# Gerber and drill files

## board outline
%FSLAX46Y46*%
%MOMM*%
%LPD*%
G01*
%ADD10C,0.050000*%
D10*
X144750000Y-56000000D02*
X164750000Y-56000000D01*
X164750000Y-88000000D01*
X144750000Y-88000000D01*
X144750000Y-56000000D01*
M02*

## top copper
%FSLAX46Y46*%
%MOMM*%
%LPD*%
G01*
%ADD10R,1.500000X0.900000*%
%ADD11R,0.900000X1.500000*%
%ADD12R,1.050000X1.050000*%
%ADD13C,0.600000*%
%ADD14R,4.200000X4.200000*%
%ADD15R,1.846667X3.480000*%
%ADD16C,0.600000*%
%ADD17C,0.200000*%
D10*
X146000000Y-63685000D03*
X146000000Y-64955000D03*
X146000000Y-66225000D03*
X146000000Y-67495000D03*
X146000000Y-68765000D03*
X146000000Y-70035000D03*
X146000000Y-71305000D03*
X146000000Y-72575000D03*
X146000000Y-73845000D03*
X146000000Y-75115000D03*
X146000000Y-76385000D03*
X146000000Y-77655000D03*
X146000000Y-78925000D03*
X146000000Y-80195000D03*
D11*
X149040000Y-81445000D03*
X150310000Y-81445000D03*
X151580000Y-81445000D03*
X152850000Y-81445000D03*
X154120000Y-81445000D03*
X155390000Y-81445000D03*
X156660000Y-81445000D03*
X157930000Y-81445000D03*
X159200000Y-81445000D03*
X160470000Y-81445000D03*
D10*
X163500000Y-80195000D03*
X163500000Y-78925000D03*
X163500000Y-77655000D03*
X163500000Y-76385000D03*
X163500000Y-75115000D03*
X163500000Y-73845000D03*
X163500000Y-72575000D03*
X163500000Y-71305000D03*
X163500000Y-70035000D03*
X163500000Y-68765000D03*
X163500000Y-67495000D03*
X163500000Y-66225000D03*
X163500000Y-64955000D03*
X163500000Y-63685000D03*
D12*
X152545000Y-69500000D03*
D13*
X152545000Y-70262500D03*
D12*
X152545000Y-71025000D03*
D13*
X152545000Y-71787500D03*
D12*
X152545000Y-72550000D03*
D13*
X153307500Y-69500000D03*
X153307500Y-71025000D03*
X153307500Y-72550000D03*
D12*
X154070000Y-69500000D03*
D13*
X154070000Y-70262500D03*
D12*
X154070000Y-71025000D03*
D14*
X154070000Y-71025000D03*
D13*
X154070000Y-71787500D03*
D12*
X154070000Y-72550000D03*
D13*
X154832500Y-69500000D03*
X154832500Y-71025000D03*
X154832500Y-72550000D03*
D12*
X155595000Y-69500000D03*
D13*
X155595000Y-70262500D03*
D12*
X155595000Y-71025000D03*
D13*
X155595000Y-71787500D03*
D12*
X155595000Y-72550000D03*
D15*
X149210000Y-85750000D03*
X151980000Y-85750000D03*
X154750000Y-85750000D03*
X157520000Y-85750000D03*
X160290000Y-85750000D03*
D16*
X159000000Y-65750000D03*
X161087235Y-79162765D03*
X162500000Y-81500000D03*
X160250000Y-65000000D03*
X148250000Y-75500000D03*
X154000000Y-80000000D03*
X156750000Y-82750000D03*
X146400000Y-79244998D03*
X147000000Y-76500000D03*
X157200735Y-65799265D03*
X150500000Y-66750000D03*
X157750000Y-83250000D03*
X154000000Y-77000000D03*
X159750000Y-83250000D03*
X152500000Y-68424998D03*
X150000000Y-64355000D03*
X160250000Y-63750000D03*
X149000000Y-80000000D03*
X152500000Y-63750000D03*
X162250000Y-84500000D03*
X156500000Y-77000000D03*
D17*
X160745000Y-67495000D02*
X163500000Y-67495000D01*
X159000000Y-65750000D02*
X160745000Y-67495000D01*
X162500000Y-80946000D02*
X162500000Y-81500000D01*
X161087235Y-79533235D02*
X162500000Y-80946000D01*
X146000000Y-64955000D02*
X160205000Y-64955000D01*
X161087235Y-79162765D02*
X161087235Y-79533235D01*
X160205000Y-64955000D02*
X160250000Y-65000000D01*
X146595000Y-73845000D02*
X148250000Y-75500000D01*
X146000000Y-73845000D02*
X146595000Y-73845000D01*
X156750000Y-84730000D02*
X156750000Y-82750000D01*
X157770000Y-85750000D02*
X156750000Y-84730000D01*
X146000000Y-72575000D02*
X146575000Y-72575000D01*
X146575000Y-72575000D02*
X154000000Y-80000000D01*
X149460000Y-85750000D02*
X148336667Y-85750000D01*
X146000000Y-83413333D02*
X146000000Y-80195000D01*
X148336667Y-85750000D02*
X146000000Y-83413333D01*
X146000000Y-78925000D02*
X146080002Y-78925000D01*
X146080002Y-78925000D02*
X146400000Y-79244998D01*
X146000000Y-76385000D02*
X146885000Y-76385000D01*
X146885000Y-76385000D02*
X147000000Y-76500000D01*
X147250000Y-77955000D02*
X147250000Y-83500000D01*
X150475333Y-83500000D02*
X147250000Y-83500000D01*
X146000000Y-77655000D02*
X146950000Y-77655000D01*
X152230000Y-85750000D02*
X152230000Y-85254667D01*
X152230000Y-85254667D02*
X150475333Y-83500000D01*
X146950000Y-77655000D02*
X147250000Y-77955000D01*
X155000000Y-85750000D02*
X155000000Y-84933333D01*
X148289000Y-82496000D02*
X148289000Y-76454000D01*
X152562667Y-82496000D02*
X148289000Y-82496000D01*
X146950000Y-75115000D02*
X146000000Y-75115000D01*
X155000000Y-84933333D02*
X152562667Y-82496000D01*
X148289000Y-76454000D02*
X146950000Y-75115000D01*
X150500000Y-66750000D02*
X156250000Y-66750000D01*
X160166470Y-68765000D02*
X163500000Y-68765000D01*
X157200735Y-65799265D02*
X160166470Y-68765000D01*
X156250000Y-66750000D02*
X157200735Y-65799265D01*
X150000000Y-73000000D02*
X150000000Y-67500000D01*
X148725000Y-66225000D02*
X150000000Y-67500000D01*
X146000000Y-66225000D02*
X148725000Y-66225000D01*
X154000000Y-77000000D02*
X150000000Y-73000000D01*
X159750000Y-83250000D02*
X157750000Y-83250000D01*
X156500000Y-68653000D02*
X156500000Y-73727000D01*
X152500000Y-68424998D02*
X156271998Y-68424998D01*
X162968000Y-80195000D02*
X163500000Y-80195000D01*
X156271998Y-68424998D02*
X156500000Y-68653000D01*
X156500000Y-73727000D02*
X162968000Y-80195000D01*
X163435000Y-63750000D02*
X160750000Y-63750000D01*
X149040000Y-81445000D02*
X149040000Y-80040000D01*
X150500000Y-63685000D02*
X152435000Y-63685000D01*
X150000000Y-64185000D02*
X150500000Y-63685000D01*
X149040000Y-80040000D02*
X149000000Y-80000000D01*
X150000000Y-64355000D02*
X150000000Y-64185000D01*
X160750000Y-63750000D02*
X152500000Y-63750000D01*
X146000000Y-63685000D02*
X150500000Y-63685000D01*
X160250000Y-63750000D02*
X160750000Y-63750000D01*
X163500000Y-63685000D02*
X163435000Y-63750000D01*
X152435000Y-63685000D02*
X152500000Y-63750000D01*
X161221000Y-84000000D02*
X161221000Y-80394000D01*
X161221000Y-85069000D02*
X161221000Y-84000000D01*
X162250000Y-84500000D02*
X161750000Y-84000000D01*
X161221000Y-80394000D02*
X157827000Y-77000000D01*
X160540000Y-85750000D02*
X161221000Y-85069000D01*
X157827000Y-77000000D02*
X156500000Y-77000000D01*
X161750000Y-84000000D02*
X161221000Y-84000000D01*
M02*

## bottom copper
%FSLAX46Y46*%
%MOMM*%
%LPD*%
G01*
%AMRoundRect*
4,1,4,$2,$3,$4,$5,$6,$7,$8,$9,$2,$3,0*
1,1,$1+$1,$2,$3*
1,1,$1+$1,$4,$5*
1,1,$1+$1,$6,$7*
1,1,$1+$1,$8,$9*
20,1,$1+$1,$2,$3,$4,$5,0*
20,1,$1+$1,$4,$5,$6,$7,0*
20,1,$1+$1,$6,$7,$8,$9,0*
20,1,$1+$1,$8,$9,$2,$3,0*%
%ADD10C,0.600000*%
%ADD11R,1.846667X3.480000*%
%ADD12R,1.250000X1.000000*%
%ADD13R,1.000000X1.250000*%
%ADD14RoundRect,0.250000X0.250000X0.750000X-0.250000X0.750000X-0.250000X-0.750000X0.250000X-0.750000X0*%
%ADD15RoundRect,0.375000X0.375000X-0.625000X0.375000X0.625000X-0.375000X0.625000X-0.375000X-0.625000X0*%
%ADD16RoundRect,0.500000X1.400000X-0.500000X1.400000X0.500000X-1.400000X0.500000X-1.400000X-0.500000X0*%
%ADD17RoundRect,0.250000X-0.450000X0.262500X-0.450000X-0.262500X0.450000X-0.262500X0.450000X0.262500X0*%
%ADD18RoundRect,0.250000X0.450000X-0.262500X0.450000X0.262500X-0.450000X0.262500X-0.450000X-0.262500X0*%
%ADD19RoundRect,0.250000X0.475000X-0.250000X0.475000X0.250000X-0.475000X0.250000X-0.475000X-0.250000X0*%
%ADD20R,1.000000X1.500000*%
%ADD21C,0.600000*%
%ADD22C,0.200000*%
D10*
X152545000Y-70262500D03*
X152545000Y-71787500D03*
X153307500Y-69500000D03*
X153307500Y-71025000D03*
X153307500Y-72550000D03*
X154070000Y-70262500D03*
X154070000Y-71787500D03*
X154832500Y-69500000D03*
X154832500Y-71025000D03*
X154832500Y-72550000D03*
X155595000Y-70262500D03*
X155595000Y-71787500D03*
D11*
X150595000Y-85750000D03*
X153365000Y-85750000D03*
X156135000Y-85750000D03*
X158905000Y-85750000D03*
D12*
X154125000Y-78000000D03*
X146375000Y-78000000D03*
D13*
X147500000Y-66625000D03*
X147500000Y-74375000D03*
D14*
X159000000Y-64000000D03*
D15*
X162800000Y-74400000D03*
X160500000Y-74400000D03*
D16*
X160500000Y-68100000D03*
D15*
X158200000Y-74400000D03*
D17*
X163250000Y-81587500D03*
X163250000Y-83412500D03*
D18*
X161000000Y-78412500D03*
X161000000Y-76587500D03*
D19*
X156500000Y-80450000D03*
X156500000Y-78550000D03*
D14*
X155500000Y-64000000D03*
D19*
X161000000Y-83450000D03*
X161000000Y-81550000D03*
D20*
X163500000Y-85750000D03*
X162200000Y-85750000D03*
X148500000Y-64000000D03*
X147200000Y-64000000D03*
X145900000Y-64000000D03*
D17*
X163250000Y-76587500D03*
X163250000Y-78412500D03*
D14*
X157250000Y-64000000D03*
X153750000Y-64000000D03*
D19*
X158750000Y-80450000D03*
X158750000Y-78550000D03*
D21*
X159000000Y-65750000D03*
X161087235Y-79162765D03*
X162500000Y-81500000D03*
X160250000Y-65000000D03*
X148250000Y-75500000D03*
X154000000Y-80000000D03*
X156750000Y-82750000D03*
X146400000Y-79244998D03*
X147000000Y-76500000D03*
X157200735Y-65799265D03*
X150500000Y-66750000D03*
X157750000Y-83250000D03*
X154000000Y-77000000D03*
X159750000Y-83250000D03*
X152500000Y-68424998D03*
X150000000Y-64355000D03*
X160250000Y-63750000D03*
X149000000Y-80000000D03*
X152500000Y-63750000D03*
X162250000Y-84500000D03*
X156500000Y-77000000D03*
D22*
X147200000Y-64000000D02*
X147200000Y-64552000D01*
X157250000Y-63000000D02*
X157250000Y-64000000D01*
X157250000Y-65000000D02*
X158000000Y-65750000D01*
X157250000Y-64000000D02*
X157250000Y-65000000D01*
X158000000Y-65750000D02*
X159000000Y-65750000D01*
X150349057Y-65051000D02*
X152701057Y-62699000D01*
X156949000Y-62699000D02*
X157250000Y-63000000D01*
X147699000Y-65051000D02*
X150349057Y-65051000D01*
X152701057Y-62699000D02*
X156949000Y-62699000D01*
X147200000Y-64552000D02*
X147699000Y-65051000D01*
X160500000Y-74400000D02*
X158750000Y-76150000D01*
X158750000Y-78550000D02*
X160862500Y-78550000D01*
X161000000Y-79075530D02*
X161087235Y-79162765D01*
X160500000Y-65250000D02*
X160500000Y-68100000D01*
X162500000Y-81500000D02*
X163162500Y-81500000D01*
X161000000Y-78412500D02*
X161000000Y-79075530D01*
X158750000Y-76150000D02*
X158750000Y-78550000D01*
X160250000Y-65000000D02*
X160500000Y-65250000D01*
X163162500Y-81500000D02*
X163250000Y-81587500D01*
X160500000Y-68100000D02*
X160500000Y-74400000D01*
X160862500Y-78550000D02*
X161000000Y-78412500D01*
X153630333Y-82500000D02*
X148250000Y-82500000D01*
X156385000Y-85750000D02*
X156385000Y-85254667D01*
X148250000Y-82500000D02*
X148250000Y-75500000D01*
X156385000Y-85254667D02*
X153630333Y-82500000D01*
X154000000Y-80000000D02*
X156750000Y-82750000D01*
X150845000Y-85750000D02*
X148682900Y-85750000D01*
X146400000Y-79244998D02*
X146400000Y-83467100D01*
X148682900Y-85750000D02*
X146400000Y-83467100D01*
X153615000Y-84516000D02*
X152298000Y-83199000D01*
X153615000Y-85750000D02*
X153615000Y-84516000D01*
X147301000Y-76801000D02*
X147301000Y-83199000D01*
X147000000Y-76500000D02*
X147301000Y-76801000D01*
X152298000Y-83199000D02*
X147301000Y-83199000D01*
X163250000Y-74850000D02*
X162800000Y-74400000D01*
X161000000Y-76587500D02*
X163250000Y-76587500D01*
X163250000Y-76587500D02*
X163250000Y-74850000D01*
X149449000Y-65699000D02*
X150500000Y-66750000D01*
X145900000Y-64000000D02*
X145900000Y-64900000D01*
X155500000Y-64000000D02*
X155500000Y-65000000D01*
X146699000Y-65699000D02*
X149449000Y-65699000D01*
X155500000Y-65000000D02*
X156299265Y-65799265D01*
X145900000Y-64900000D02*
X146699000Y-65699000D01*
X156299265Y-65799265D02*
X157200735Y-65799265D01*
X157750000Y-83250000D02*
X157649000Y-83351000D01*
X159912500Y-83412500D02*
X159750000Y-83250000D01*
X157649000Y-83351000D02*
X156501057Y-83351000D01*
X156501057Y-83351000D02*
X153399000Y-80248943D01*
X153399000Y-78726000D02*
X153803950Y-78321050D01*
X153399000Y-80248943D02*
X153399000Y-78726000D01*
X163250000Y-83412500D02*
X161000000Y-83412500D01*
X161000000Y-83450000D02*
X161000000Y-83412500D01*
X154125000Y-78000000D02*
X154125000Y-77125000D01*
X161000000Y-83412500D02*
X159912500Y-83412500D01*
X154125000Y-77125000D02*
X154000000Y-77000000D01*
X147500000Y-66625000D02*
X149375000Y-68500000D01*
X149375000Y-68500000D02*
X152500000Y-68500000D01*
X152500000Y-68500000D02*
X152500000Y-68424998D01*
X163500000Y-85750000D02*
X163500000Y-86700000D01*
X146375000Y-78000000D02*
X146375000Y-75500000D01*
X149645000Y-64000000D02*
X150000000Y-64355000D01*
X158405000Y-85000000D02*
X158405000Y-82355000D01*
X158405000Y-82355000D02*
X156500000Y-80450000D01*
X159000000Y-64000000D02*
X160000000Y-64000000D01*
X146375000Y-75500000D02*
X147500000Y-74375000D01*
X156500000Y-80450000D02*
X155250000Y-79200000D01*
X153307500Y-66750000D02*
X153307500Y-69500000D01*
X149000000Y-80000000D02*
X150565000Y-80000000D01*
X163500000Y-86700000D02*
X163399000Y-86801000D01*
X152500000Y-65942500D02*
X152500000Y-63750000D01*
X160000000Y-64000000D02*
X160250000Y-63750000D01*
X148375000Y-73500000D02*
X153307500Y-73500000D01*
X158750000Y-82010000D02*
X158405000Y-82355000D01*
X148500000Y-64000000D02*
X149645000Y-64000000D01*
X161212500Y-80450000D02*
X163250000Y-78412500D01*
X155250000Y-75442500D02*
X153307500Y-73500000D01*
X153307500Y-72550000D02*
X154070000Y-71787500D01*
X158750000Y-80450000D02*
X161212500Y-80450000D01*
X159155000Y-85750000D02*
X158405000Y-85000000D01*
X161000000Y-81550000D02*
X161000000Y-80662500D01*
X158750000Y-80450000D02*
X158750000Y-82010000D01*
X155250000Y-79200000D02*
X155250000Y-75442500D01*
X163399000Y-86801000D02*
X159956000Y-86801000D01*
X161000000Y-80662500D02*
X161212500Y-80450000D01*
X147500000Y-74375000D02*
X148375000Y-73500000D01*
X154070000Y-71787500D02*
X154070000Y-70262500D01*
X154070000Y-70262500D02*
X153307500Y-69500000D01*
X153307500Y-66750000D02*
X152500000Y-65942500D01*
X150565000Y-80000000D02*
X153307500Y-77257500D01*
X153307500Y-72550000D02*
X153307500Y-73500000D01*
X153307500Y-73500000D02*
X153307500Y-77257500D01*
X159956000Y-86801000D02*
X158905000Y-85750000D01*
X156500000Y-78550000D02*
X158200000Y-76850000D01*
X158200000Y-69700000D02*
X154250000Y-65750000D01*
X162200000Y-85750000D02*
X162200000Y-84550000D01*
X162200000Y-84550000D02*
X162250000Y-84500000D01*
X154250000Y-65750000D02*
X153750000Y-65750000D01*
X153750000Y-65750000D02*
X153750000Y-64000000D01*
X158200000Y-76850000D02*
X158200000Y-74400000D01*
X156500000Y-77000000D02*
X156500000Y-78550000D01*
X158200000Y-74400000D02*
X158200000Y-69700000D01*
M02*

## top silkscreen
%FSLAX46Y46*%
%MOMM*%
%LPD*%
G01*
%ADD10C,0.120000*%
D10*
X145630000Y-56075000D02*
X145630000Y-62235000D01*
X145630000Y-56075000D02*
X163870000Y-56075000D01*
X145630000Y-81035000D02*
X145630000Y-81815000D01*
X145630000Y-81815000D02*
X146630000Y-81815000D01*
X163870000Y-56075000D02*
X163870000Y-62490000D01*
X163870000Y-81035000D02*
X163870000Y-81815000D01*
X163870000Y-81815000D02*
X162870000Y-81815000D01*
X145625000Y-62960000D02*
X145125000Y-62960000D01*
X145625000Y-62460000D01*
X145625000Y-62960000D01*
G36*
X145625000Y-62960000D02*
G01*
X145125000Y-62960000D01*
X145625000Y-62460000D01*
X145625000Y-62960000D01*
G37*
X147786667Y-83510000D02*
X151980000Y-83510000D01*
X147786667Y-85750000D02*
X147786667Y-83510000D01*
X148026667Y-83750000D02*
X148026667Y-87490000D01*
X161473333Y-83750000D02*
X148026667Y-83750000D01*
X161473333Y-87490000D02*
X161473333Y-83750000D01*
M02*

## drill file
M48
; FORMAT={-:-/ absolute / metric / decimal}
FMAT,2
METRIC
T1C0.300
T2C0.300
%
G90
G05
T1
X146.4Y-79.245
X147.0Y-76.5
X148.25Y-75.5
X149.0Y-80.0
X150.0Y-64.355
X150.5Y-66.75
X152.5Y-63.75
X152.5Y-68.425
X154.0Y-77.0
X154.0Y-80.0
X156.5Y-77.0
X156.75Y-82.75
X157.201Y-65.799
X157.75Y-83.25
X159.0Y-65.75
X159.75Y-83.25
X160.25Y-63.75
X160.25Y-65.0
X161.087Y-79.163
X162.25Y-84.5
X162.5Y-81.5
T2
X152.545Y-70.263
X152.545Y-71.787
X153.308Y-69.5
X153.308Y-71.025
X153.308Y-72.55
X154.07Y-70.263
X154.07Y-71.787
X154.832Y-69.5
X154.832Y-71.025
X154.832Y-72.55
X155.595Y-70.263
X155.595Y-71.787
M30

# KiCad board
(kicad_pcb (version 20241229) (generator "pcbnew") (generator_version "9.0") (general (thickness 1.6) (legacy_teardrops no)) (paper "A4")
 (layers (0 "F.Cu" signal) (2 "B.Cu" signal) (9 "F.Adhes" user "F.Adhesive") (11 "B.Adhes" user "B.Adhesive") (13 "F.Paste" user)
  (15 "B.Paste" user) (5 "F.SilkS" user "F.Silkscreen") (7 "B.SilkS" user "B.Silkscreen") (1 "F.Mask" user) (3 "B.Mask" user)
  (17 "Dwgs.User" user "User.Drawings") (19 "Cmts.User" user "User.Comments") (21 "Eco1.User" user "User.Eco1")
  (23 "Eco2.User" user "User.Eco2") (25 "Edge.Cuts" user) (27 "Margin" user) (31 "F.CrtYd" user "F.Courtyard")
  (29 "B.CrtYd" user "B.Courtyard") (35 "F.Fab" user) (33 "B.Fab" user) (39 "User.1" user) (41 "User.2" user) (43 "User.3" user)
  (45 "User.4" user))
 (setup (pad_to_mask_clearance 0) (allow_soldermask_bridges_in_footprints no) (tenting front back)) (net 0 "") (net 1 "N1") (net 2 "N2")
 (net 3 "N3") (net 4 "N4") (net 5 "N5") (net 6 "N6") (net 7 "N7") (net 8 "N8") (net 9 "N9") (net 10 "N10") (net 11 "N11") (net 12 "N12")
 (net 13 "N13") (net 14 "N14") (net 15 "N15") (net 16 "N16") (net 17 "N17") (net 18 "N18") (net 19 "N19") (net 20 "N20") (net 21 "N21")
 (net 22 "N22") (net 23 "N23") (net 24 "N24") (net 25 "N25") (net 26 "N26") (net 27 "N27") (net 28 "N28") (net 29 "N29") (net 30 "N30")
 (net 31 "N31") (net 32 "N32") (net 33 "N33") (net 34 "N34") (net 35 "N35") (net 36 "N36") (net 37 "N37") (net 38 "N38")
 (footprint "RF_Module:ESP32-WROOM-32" (layer "F.Cu") (at 154.75 71.935)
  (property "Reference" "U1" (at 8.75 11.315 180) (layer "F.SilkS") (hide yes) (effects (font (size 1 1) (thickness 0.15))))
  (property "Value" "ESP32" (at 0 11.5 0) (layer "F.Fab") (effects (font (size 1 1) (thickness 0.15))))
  (fp_line (start -9.12 -15.86) (end -9.12 -9.7) (stroke (width 0.12) (type solid)) (layer "F.SilkS"))
  (fp_line (start -9.12 -15.86) (end 9.12 -15.86) (stroke (width 0.12) (type solid)) (layer "F.SilkS"))
  (fp_line (start -9.12 9.1) (end -9.12 9.88) (stroke (width 0.12) (type solid)) (layer "F.SilkS"))
  (fp_line (start -9.12 9.88) (end -8.12 9.88) (stroke (width 0.12) (type solid)) (layer "F.SilkS"))
  (fp_line (start 9.12 -15.86) (end 9.12 -9.445) (stroke (width 0.12) (type solid)) (layer "F.SilkS"))
  (fp_line (start 9.12 9.1) (end 9.12 9.88) (stroke (width 0.12) (type solid)) (layer "F.SilkS"))
  (fp_line (start 9.12 9.88) (end 8.12 9.88) (stroke (width 0.12) (type solid)) (layer "F.SilkS"))
  (fp_poly
   (pts (xy -9.125 -8.975) (xy -9.625 -8.975) (xy -9.125 -9.475) (xy -9.125 -8.975)) (stroke (width 0.12) (type solid)) (fill yes)
   (layer "F.SilkS"))
  (pad "1" smd rect (at -8.75 -8.25) (size 1.5 0.9) (layers "F.Cu" "F.Mask" "F.Paste") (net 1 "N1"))
  (pad "2" smd rect (at -8.75 -6.98) (size 1.5 0.9) (layers "F.Cu" "F.Mask" "F.Paste") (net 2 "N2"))
  (pad "3" smd rect (at -8.75 -5.71) (size 1.5 0.9) (layers "F.Cu" "F.Mask" "F.Paste") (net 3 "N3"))
  (pad "4" smd rect (at -8.75 -4.44) (size 1.5 0.9) (layers "F.Cu" "F.Mask" "F.Paste") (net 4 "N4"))
  (pad "5" smd rect (at -8.75 -3.17) (size 1.5 0.9) (layers "F.Cu" "F.Mask" "F.Paste") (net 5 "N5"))
  (pad "6" smd rect (at -8.75 -1.9) (size 1.5 0.9) (layers "F.Cu" "F.Mask" "F.Paste") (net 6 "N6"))
  (pad "7" smd rect (at -8.75 -0.63) (size 1.5 0.9) (layers "F.Cu" "F.Mask" "F.Paste") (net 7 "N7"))
  (pad "8" smd rect (at -8.75 0.64) (size 1.5 0.9) (layers "F.Cu" "F.Mask" "F.Paste") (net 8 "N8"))
  (pad "9" smd rect (at -8.75 1.91) (size 1.5 0.9) (layers "F.Cu" "F.Mask" "F.Paste") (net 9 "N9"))
  (pad "10" smd rect (at -8.75 3.18) (size 1.5 0.9) (layers "F.Cu" "F.Mask" "F.Paste") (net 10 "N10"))
  (pad "11" smd rect (at -8.75 4.45) (size 1.5 0.9) (layers "F.Cu" "F.Mask" "F.Paste") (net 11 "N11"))
  (pad "12" smd rect (at -8.75 5.72) (size 1.5 0.9) (layers "F.Cu" "F.Mask" "F.Paste") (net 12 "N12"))
  (pad "13" smd rect (at -8.75 6.99) (size 1.5 0.9) (layers "F.Cu" "F.Mask" "F.Paste") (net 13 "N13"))
  (pad "14" smd rect (at -8.75 8.26) (size 1.5 0.9) (layers "F.Cu" "F.Mask" "F.Paste") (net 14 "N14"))
  (pad "15" smd rect (at -5.71 9.51 90) (size 1.5 0.9) (layers "F.Cu" "F.Mask" "F.Paste") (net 1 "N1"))
  (pad "16" smd rect (at -4.44 9.51 90) (size 1.5 0.9) (layers "F.Cu" "F.Mask" "F.Paste") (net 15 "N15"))
  (pad "17" smd rect (at -3.17 9.51 90) (size 1.5 0.9) (layers "F.Cu" "F.Mask" "F.Paste") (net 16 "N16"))
  (pad "18" smd rect (at -1.9 9.51 90) (size 1.5 0.9) (layers "F.Cu" "F.Mask" "F.Paste") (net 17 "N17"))
  (pad "19" smd rect (at -0.63 9.51 90) (size 1.5 0.9) (layers "F.Cu" "F.Mask" "F.Paste") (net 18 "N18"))
  (pad "20" smd rect (at 0.64 9.51 90) (size 1.5 0.9) (layers "F.Cu" "F.Mask" "F.Paste") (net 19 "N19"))
  (pad "21" smd rect (at 1.91 9.51 90) (size 1.5 0.9) (layers "F.Cu" "F.Mask" "F.Paste") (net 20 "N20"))
  (pad "22" smd rect (at 3.18 9.51 90) (size 1.5 0.9) (layers "F.Cu" "F.Mask" "F.Paste") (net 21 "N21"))
  (pad "23" smd rect (at 4.45 9.51 90) (size 1.5 0.9) (layers "F.Cu" "F.Mask" "F.Paste") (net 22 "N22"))
  (pad "24" smd rect (at 5.72 9.51 90) (size 1.5 0.9) (layers "F.Cu" "F.Mask" "F.Paste") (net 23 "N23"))
  (pad "25" smd rect (at 8.75 8.26) (size 1.5 0.9) (layers "F.Cu" "F.Mask" "F.Paste") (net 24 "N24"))
  (pad "26" smd rect (at 8.75 6.99) (size 1.5 0.9) (layers "F.Cu" "F.Mask" "F.Paste") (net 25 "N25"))
  (pad "27" smd rect (at 8.75 5.72) (size 1.5 0.9) (layers "F.Cu" "F.Mask" "F.Paste") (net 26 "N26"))
  (pad "28" smd rect (at 8.75 4.45) (size 1.5 0.9) (layers "F.Cu" "F.Mask" "F.Paste") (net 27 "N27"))
  (pad "29" smd rect (at 8.75 3.18) (size 1.5 0.9) (layers "F.Cu" "F.Mask" "F.Paste") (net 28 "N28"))
  (pad "30" smd rect (at 8.75 1.91) (size 1.5 0.9) (layers "F.Cu" "F.Mask" "F.Paste") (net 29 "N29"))
  (pad "31" smd rect (at 8.75 0.64) (size 1.5 0.9) (layers "F.Cu" "F.Mask" "F.Paste") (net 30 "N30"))
  (pad "32" smd rect (at 8.75 -0.63) (size 1.5 0.9) (layers "F.Cu" "F.Mask" "F.Paste") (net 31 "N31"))
  (pad "33" smd rect (at 8.75 -1.9) (size 1.5 0.9) (layers "F.Cu" "F.Mask" "F.Paste") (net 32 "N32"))
  (pad "34" smd rect (at 8.75 -3.17) (size 1.5 0.9) (layers "F.Cu" "F.Mask" "F.Paste") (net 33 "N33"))
  (pad "35" smd rect (at 8.75 -4.44) (size 1.5 0.9) (layers "F.Cu" "F.Mask" "F.Paste") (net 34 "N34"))
  (pad "36" smd rect (at 8.75 -5.71) (size 1.5 0.9) (layers "F.Cu" "F.Mask" "F.Paste") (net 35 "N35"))
  (pad "37" smd rect (at 8.75 -6.98) (size 1.5 0.9) (layers "F.Cu" "F.Mask" "F.Paste") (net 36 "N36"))
  (pad "38" smd rect (at 8.75 -8.25) (size 1.5 0.9) (layers "F.Cu" "F.Mask" "F.Paste") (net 1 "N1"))
  (pad "39" smd rect (at -2.205 -2.435) (size 1.05 1.05) (layers "F.Cu" "F.Paste") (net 1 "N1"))
  (pad "39" thru_hole circle (at -2.205 -1.6725) (size 0.6 0.6) (drill 0.3) (layers "*.Cu" "F.Mask") (remove_unused_layers no) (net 1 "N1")
   (zone_connect 2))
  (pad "39" smd rect (at -2.205 -0.91) (size 1.05 1.05) (layers "F.Cu" "F.Paste") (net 1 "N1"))
  (pad "39" thru_hole circle (at -2.205 -0.1475) (size 0.6 0.6) (drill 0.3) (layers "*.Cu" "F.Mask") (remove_unused_layers no) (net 1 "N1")
   (zone_connect 2))
  (pad "39" smd rect (at -2.205 0.615) (size 1.05 1.05) (layers "F.Cu" "F.Paste") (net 1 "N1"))
  (pad "39" thru_hole circle (at -1.4425 -2.435) (size 0.6 0.6) (drill 0.3) (layers "*.Cu" "F.Mask") (remove_unused_layers no) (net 1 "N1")
   (zone_connect 2))
  (pad "39" thru_hole circle (at -1.4425 -0.91) (size 0.6 0.6) (drill 0.3) (layers "*.Cu" "F.Mask") (remove_unused_layers no) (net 1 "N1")
   (zone_connect 2))
  (pad "39" thru_hole circle (at -1.4425 0.615) (size 0.6 0.6) (drill 0.3) (layers "*.Cu" "F.Mask") (remove_unused_layers no) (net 1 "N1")
   (zone_connect 2))
  (pad "39" smd rect (at -0.68 -2.435) (size 1.05 1.05) (layers "F.Cu" "F.Paste") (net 1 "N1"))
  (pad "39" thru_hole circle (at -0.68 -1.6725) (size 0.6 0.6) (drill 0.3) (layers "*.Cu" "F.Mask") (remove_unused_layers no) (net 1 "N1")
   (zone_connect 2))
  (pad "39" smd rect (at -0.68 -0.91) (size 1.05 1.05) (layers "F.Cu" "F.Paste") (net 1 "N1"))
  (pad "39" smd rect (at -0.68 -0.91) (size 4.2 4.2) (layers "F.Cu" "F.Mask") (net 1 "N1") (zone_connect 2))
  (pad "39" thru_hole circle (at -0.68 -0.1475) (size 0.6 0.6) (drill 0.3) (layers "*.Cu" "F.Mask") (remove_unused_layers no) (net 1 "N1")
   (zone_connect 2))
  (pad "39" smd rect (at -0.68 0.615) (size 1.05 1.05) (layers "F.Cu" "F.Paste") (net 1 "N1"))
  (pad "39" thru_hole circle (at 0.0825 -2.435) (size 0.6 0.6) (drill 0.3) (layers "*.Cu" "F.Mask") (remove_unused_layers no) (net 1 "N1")
   (zone_connect 2))
  (pad "39" thru_hole circle (at 0.0825 -0.91) (size 0.6 0.6) (drill 0.3) (layers "*.Cu" "F.Mask") (remove_unused_layers no) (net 1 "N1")
   (zone_connect 2))
  (pad "39" thru_hole circle (at 0.0825 0.615) (size 0.6 0.6) (drill 0.3) (layers "*.Cu" "F.Mask") (remove_unused_layers no) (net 1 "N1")
   (zone_connect 2))
  (pad "39" smd rect (at 0.845 -2.435) (size 1.05 1.05) (layers "F.Cu" "F.Paste") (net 1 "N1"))
  (pad "39" thru_hole circle (at 0.845 -1.6725) (size 0.6 0.6) (drill 0.3) (layers "*.Cu" "F.Mask") (remove_unused_layers no) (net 1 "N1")
   (zone_connect 2))
  (pad "39" smd rect (at 0.845 -0.91) (size 1.05 1.05) (layers "F.Cu" "F.Paste") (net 1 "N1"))
  (pad "39" thru_hole circle (at 0.845 -0.1475) (size 0.6 0.6) (drill 0.3) (layers "*.Cu" "F.Mask") (remove_unused_layers no) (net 1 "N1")
   (zone_connect 2))
  (pad "39" smd rect (at 0.845 0.615) (size 1.05 1.05) (layers "F.Cu" "F.Paste") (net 1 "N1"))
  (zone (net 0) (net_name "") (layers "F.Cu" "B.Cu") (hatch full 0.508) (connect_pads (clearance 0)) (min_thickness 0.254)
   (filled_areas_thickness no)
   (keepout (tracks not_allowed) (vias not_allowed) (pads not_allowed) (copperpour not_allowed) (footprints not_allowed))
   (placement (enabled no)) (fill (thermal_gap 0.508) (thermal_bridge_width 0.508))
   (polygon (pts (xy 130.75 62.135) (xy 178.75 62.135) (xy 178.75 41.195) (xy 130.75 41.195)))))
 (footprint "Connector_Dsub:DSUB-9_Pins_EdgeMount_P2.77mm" (layer "F.Cu") (at 154.75 85.75)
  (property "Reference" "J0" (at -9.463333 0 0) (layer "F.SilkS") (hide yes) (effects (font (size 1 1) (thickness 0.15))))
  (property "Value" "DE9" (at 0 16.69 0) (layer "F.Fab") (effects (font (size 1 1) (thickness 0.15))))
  (fp_line (start -6.963333 -2.24) (end -2.77 -2.24) (stroke (width 0.12) (type solid)) (layer "F.SilkS"))
  (fp_line (start -6.963333 0) (end -6.963333 -2.24) (stroke (width 0.12) (type solid)) (layer "F.SilkS"))
  (fp_line (start -6.723333 -2) (end -6.723333 1.74) (stroke (width 0.12) (type solid)) (layer "F.SilkS"))
  (fp_line (start 6.723333 -2) (end -6.723333 -2) (stroke (width 0.12) (type solid)) (layer "F.SilkS"))
  (fp_line (start 6.723333 1.74) (end 6.723333 -2) (stroke (width 0.12) (type solid)) (layer "F.SilkS"))
  (pad "1" smd rect (at -5.54 0) (size 1.846667 3.48) (layers "F.Cu" "F.Mask" "F.Paste") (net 14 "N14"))
  (pad "2" smd rect (at -2.77 0) (size 1.846667 3.48) (layers "F.Cu" "F.Mask" "F.Paste") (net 12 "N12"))
  (pad "3" smd rect (at 0 0) (size 1.846667 3.48) (layers "F.Cu" "F.Mask" "F.Paste") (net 10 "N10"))
  (pad "4" smd rect (at 2.77 0) (size 1.846667 3.48) (layers "F.Cu" "F.Mask" "F.Paste") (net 8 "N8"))
  (pad "5" smd rect (at 5.54 0) (size 1.846667 3.48) (layers "F.Cu" "F.Mask" "F.Paste") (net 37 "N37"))
  (pad "6" smd rect (at -4.155 0) (size 1.846667 3.48) (layers "B.Cu" "B.Mask" "B.Paste") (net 13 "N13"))
  (pad "7" smd rect (at -1.385 0) (size 1.846667 3.48) (layers "B.Cu" "B.Mask" "B.Paste") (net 11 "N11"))
  (pad "8" smd rect (at 1.385 0) (size 1.846667 3.48) (layers "B.Cu" "B.Mask" "B.Paste") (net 9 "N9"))
  (pad "9" smd rect (at 4.155 0) (size 1.846667 3.48) (layers "B.Cu" "B.Mask" "B.Paste") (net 1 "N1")))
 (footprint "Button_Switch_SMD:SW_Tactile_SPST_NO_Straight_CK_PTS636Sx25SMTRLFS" (layer "B.Cu") (at 150.25 78 180)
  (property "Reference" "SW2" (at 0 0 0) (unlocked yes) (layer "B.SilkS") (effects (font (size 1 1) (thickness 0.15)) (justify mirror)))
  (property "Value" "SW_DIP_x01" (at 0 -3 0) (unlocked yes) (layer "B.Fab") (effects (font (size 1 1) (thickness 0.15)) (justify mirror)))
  (pad "1" smd rect (at -3.875 0 180) (size 1.25 1) (layers "B.Cu" "B.Mask" "B.Paste") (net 3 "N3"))
  (pad "2" smd rect (at 3.875 0 180) (size 1.25 1) (layers "B.Cu" "B.Mask" "B.Paste") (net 1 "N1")))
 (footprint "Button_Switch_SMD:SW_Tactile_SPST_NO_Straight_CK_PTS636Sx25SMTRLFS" (layer "B.Cu") (at 147.5 70.5 -90)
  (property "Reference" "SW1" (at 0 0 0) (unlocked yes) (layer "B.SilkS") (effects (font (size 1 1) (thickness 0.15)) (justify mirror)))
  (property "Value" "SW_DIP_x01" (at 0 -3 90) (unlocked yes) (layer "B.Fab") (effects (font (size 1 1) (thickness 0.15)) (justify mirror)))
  (pad "1" smd rect (at -3.875 0 270) (size 1.25 1) (layers "B.Cu" "B.Mask" "B.Paste") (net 24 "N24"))
  (pad "2" smd rect (at 3.875 0 270) (size 1.25 1) (layers "B.Cu" "B.Mask" "B.Paste") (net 1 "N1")))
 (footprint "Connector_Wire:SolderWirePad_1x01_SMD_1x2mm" (layer "B.Cu") (at 159 64 180)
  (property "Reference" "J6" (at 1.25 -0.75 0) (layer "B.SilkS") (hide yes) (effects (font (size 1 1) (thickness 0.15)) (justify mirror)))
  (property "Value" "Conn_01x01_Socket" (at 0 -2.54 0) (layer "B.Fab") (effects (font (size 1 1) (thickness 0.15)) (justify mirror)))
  (pad "1" smd roundrect (at 0 0 180) (size 1 2) (layers "B.Cu" "B.Mask") (roundrect_rratio 0.25) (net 1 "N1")))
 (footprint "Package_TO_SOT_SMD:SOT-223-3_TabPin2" (layer "B.Cu") (at 160.5 71.25 90)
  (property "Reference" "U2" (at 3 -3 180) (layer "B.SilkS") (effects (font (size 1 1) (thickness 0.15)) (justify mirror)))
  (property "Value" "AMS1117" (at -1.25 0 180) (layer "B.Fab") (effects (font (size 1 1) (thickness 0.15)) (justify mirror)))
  (pad "1" smd roundrect (at -3.15 2.3 90) (size 2 1.5) (layers "B.Cu" "B.Mask" "B.Paste") (roundrect_rratio 0.25) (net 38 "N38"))
  (pad "2" smd roundrect (at -3.15 0 90) (size 2 1.5) (layers "B.Cu" "B.Mask" "B.Paste") (roundrect_rratio 0.25) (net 2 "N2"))
  (pad "2" smd roundrect (at 3.15 0 90) (size 2 3.8) (layers "B.Cu" "B.Mask" "B.Paste") (roundrect_rratio 0.25) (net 2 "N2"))
  (pad "3" smd roundrect (at -3.15 -2.3 90) (size 2 1.5) (layers "B.Cu" "B.Mask" "B.Paste") (roundrect_rratio 0.25) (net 37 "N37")))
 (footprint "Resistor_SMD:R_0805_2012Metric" (layer "B.Cu") (at 163.25 82.5 -90)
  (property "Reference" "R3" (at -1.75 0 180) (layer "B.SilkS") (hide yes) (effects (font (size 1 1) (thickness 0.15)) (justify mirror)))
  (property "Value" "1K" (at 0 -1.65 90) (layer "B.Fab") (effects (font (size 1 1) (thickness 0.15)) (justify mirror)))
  (pad "1" smd roundrect (at -0.9125 0 270) (size 1.025 1.4) (layers "B.Cu" "B.Mask" "B.Paste") (roundrect_rratio 0.243902) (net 2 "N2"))
  (pad "2" smd roundrect (at 0.9125 0 270) (size 1.025 1.4) (layers "B.Cu" "B.Mask" "B.Paste") (roundrect_rratio 0.243902) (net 3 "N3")))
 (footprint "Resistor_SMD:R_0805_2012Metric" (layer "B.Cu") (at 161 77.5 90)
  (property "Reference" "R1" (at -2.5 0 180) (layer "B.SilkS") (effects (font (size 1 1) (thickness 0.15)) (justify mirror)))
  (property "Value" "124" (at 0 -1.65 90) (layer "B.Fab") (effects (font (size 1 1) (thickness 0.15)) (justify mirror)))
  (pad "1" smd roundrect (at -0.9125 0 90) (size 1.025 1.4) (layers "B.Cu" "B.Mask" "B.Paste") (roundrect_rratio 0.243902) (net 2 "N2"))
  (pad "2" smd roundrect (at 0.9125 0 90) (size 1.025 1.4) (layers "B.Cu" "B.Mask" "B.Paste") (roundrect_rratio 0.243902) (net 38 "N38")))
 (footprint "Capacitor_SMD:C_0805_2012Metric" (layer "B.Cu") (at 156.5 79.5 90)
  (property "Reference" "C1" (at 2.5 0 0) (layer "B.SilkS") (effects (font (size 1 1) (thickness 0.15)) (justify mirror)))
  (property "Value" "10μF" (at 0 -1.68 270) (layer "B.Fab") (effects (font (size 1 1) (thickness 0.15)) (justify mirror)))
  (pad "1" smd roundrect (at -0.95 0 90) (size 1 1.45) (layers "B.Cu" "B.Mask" "B.Paste") (roundrect_rratio 0.25) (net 1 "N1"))
  (pad "2" smd roundrect (at 0.95 0 90) (size 1 1.45) (layers "B.Cu" "B.Mask" "B.Paste") (roundrect_rratio 0.25) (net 37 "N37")))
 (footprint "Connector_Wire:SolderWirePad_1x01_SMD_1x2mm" (layer "B.Cu") (at 155.5 64 180)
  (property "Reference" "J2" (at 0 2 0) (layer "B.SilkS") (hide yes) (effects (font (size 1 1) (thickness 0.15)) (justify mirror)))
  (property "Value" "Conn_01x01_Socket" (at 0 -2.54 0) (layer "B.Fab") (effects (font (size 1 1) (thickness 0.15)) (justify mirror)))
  (pad "1" smd roundrect (at 0 0 180) (size 1 2) (layers "B.Cu" "B.Mask") (roundrect_rratio 0.25) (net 33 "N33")))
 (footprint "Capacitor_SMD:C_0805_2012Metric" (layer "B.Cu") (at 161 82.5 90)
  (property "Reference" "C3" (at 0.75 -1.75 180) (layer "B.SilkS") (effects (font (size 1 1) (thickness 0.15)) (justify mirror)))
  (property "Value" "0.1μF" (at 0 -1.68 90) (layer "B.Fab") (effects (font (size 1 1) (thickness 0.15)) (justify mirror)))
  (pad "1" smd roundrect (at -0.95 0 90) (size 1 1.45) (layers "B.Cu" "B.Mask" "B.Paste") (roundrect_rratio 0.25) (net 3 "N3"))
  (pad "2" smd roundrect (at 0.95 0 90) (size 1 1.45) (layers "B.Cu" "B.Mask" "B.Paste") (roundrect_rratio 0.25) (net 1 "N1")))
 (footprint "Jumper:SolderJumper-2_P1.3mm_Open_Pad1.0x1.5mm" (layer "B.Cu") (at 162.85 85.75 180)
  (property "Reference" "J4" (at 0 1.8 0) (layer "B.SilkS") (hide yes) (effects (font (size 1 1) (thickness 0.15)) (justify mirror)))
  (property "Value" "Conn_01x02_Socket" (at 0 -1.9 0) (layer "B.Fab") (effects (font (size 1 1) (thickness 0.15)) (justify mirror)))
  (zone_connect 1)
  (pad "1" smd rect (at -0.65 0 180) (size 1 1.5) (layers "B.Cu" "B.Mask") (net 1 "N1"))
  (pad "2" smd rect (at 0.65 0 180) (size 1 1.5) (layers "B.Cu" "B.Mask") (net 37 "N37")))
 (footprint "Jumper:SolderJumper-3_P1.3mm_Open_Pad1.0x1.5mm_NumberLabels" (layer "B.Cu") (at 147.2 64 180)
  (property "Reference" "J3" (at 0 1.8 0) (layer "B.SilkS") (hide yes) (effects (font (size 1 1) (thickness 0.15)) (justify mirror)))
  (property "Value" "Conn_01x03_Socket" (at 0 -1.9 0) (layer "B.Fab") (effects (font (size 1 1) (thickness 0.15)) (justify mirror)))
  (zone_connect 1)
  (pad "1" smd rect (at -1.3 0 180) (size 1 1.5) (layers "B.Cu" "B.Mask") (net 1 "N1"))
  (pad "2" smd rect (at 0 0 180) (size 1 1.5) (layers "B.Cu" "B.Mask") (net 34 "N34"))
  (pad "3" smd rect (at 1.3 0 180) (size 1 1.5) (layers "B.Cu" "B.Mask") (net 33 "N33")))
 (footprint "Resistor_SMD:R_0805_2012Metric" (layer "B.Cu") (at 163.25 77.5 -90)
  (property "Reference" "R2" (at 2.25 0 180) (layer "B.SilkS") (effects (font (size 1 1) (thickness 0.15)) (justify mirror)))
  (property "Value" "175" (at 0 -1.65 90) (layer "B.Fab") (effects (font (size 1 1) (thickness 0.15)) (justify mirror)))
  (pad "1" smd roundrect (at -0.9125 0 270) (size 1.025 1.4) (layers "B.Cu" "B.Mask" "B.Paste") (roundrect_rratio 0.243902) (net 38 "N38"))
  (pad "2" smd roundrect (at 0.9125 0 270) (size 1.025 1.4) (layers "B.Cu" "B.Mask" "B.Paste") (roundrect_rratio 0.243902) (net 1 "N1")))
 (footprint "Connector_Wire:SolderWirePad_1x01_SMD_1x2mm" (layer "B.Cu") (at 157.25 64 180)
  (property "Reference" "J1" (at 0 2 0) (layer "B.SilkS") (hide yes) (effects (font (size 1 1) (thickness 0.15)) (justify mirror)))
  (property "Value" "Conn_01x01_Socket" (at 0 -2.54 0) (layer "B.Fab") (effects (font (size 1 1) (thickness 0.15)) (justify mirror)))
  (pad "1" smd roundrect (at 0 0 180) (size 1 2) (layers "B.Cu" "B.Mask") (roundrect_rratio 0.25) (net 34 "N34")))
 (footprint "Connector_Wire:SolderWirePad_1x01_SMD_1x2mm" (layer "B.Cu") (at 153.75 64 180)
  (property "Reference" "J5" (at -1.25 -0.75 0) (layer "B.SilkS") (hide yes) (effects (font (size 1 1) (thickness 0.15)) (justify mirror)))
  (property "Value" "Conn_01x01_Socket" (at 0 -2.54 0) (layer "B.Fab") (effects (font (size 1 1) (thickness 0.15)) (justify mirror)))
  (pad "1" smd roundrect (at 0 0 180) (size 1 2) (layers "B.Cu" "B.Mask") (roundrect_rratio 0.25) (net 37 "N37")))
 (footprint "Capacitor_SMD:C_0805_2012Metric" (layer "B.Cu") (at 158.75 79.5 90)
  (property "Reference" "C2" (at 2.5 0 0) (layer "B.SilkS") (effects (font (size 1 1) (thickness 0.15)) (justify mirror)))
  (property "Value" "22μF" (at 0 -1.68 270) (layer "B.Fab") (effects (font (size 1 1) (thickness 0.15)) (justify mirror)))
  (pad "1" smd roundrect (at -0.95 0 90) (size 1 1.45) (layers "B.Cu" "B.Mask" "B.Paste") (roundrect_rratio 0.25) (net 1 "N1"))
  (pad "2" smd roundrect (at 0.95 0 90) (size 1 1.45) (layers "B.Cu" "B.Mask" "B.Paste") (roundrect_rratio 0.25) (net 2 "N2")))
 (gr_rect (start 144.75 56) (end 164.75 88) (stroke (width 0.05) (type default)) (fill no) (layer "Edge.Cuts"))
 (segment (start 160.745 67.495) (end 163.5 67.495) (width 0.2) (layer "F.Cu") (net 34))
 (segment (start 159 65.75) (end 160.745 67.495) (width 0.2) (layer "F.Cu") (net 34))
 (via (at 159 65.75) (size 0.6) (drill 0.3) (layers "F.Cu" "B.Cu") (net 34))
 (segment (start 147.2 64) (end 147.2 64.552) (width 0.2) (layer "B.Cu") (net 34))
 (segment (start 157.25 63) (end 157.25 64) (width 0.2) (layer "B.Cu") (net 34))
 (segment (start 157.25 65) (end 158 65.75) (width 0.2) (layer "B.Cu") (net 34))
 (segment (start 157.25 64) (end 157.25 65) (width 0.2) (layer "B.Cu") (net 34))
 (segment (start 158 65.75) (end 159 65.75) (width 0.2) (layer "B.Cu") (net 34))
 (segment (start 150.349057 65.051) (end 152.701057 62.699) (width 0.2) (layer "B.Cu") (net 34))
 (segment (start 156.949 62.699) (end 157.25 63) (width 0.2) (layer "B.Cu") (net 34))
 (segment (start 147.699 65.051) (end 150.349057 65.051) (width 0.2) (layer "B.Cu") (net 34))
 (segment (start 152.701057 62.699) (end 156.949 62.699) (width 0.2) (layer "B.Cu") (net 34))
 (segment (start 147.2 64.552) (end 147.699 65.051) (width 0.2) (layer "B.Cu") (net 34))
 (segment (start 162.5 80.946) (end 162.5 81.5) (width 0.2) (layer "F.Cu") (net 2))
 (segment (start 161.087235 79.533235) (end 162.5 80.946) (width 0.2) (layer "F.Cu") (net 2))
 (segment (start 146 64.955) (end 160.205 64.955) (width 0.2) (layer "F.Cu") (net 2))
 (segment (start 161.087235 79.162765) (end 161.087235 79.533235) (width 0.2) (layer "F.Cu") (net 2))
 (segment (start 160.205 64.955) (end 160.25 65) (width 0.2) (layer "F.Cu") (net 2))
 (via (at 161.087235 79.162765) (size 0.6) (drill 0.3) (layers "F.Cu" "B.Cu") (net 2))
 (via (at 162.5 81.5) (size 0.6) (drill 0.3) (layers "F.Cu" "B.Cu") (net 2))
 (via (at 160.25 65) (size 0.6) (drill 0.3) (layers "F.Cu" "B.Cu") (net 2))
 (segment (start 160.5 74.4) (end 158.75 76.15) (width 0.2) (layer "B.Cu") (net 2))
 (segment (start 158.75 78.55) (end 160.8625 78.55) (width 0.2) (layer "B.Cu") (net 2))
 (segment (start 161 79.07553) (end 161.087235 79.162765) (width 0.2) (layer "B.Cu") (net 2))
 (segment (start 160.5 65.25) (end 160.5 68.1) (width 0.2) (layer "B.Cu") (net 2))
 (segment (start 162.5 81.5) (end 163.1625 81.5) (width 0.2) (layer "B.Cu") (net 2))
 (segment (start 161 78.4125) (end 161 79.07553) (width 0.2) (layer "B.Cu") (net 2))
 (segment (start 158.75 76.15) (end 158.75 78.55) (width 0.2) (layer "B.Cu") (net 2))
 (segment (start 160.25 65) (end 160.5 65.25) (width 0.2) (layer "B.Cu") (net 2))
 (segment (start 163.1625 81.5) (end 163.25 81.5875) (width 0.2) (layer "B.Cu") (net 2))
 (segment (start 160.5 68.1) (end 160.5 74.4) (width 0.2) (layer "B.Cu") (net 2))
 (segment (start 160.8625 78.55) (end 161 78.4125) (width 0.2) (layer "B.Cu") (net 2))
 (segment (start 146.595 73.845) (end 148.25 75.5) (width 0.2) (layer "F.Cu") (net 9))
 (segment (start 146 73.845) (end 146.595 73.845) (width 0.2) (layer "F.Cu") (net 9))
 (via (at 148.25 75.5) (size 0.6) (drill 0.3) (layers "F.Cu" "B.Cu") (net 9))
 (segment (start 153.630333 82.5) (end 148.25 82.5) (width 0.2) (layer "B.Cu") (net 9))
 (segment (start 156.385 85.75) (end 156.385 85.254667) (width 0.2) (layer "B.Cu") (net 9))
 (segment (start 148.25 82.5) (end 148.25 75.5) (width 0.2) (layer "B.Cu") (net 9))
 (segment (start 156.385 85.254667) (end 153.630333 82.5) (width 0.2) (layer "B.Cu") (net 9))
 (segment (start 156.75 84.73) (end 156.75 82.75) (width 0.2) (layer "F.Cu") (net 8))
 (segment (start 157.77 85.75) (end 156.75 84.73) (width 0.2) (layer "F.Cu") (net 8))
 (segment (start 146 72.575) (end 146.575 72.575) (width 0.2) (layer "F.Cu") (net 8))
 (segment (start 146.575 72.575) (end 154 80) (width 0.2) (layer "F.Cu") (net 8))
 (via (at 154 80) (size 0.6) (drill 0.3) (layers "F.Cu" "B.Cu") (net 8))
 (via (at 156.75 82.75) (size 0.6) (drill 0.3) (layers "F.Cu" "B.Cu") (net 8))
 (segment (start 154 80) (end 156.75 82.75) (width 0.2) (layer "B.Cu") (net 8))
 (segment (start 149.46 85.75) (end 148.336667 85.75) (width 0.2) (layer "F.Cu") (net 14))
 (segment (start 146 83.413333) (end 146 80.195) (width 0.2) (layer "F.Cu") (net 14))
 (segment (start 148.336667 85.75) (end 146 83.413333) (width 0.2) (layer "F.Cu") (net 14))
 (segment (start 146 78.925) (end 146.080002 78.925) (width 0.2) (layer "F.Cu") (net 13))
 (segment (start 146.080002 78.925) (end 146.4 79.244998) (width 0.2) (layer "F.Cu") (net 13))
 (via (at 146.4 79.244998) (size 0.6) (drill 0.3) (layers "F.Cu" "B.Cu") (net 13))
 (segment (start 150.845 85.75) (end 148.6829 85.75) (width 0.2) (layer "B.Cu") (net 13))
 (segment (start 146.4 79.244998) (end 146.4 83.4671) (width 0.2) (layer "B.Cu") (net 13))
 (segment (start 148.6829 85.75) (end 146.4 83.4671) (width 0.2) (layer "B.Cu") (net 13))
 (segment (start 146 76.385) (end 146.885 76.385) (width 0.2) (layer "F.Cu") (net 11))
 (segment (start 146.885 76.385) (end 147 76.5) (width 0.2) (layer "F.Cu") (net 11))
 (via (at 147 76.5) (size 0.6) (drill 0.3) (layers "F.Cu" "B.Cu") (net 11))
 (segment (start 153.615 84.516) (end 152.298 83.199) (width 0.2) (layer "B.Cu") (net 11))
 (segment (start 153.615 85.75) (end 153.615 84.516) (width 0.2) (layer "B.Cu") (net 11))
 (segment (start 147.301 76.801) (end 147.301 83.199) (width 0.2) (layer "B.Cu") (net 11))
 (segment (start 147 76.5) (end 147.301 76.801) (width 0.2) (layer "B.Cu") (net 11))
 (segment (start 152.298 83.199) (end 147.301 83.199) (width 0.2) (layer "B.Cu") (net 11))
 (segment (start 147.25 77.955) (end 147.25 83.5) (width 0.2) (layer "F.Cu") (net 12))
 (segment (start 150.475333 83.5) (end 147.25 83.5) (width 0.2) (layer "F.Cu") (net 12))
 (segment (start 146 77.655) (end 146.95 77.655) (width 0.2) (layer "F.Cu") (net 12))
 (segment (start 152.23 85.75) (end 152.23 85.254667) (width 0.2) (layer "F.Cu") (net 12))
 (segment (start 152.23 85.254667) (end 150.475333 83.5) (width 0.2) (layer "F.Cu") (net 12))
 (segment (start 146.95 77.655) (end 147.25 77.955) (width 0.2) (layer "F.Cu") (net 12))
 (segment (start 155 85.75) (end 155 84.933333) (width 0.2) (layer "F.Cu") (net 10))
 (segment (start 148.289 82.496) (end 148.289 76.454) (width 0.2) (layer "F.Cu") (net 10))
 (segment (start 152.562667 82.496) (end 148.289 82.496) (width 0.2) (layer "F.Cu") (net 10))
 (segment (start 146.95 75.115) (end 146 75.115) (width 0.2) (layer "F.Cu") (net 10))
 (segment (start 155 84.933333) (end 152.562667 82.496) (width 0.2) (layer "F.Cu") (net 10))
 (segment (start 148.289 76.454) (end 146.95 75.115) (width 0.2) (layer "F.Cu") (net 10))
 (segment (start 163.25 74.85) (end 162.8 74.4) (width 0.2) (layer "B.Cu") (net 38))
 (segment (start 161 76.5875) (end 163.25 76.5875) (width 0.2) (layer "B.Cu") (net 38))
 (segment (start 163.25 76.5875) (end 163.25 74.85) (width 0.2) (layer "B.Cu") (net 38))
 (segment (start 150.5 66.75) (end 156.25 66.75) (width 0.2) (layer "F.Cu") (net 33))
 (segment (start 160.16647 68.765) (end 163.5 68.765) (width 0.2) (layer "F.Cu") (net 33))
 (segment (start 157.200735 65.799265) (end 160.16647 68.765) (width 0.2) (layer "F.Cu") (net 33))
 (segment (start 156.25 66.75) (end 157.200735 65.799265) (width 0.2) (layer "F.Cu") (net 33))
 (via (at 157.200735 65.799265) (size 0.6) (drill 0.3) (layers "F.Cu" "B.Cu") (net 33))
 (via (at 150.5 66.75) (size 0.6) (drill 0.3) (layers "F.Cu" "B.Cu") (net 33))
 (segment (start 149.449 65.699) (end 150.5 66.75) (width 0.2) (layer "B.Cu") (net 33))
 (segment (start 145.9 64) (end 145.9 64.9) (width 0.2) (layer "B.Cu") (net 33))
 (segment (start 155.5 64) (end 155.5 65) (width 0.2) (layer "B.Cu") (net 33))
 (segment (start 146.699 65.699) (end 149.449 65.699) (width 0.2) (layer "B.Cu") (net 33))
 (segment (start 155.5 65) (end 156.299265 65.799265) (width 0.2) (layer "B.Cu") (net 33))
 (segment (start 145.9 64.9) (end 146.699 65.699) (width 0.2) (layer "B.Cu") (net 33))
 (segment (start 156.299265 65.799265) (end 157.200735 65.799265) (width 0.2) (layer "B.Cu") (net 33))
 (segment (start 150 73) (end 150 67.5) (width 0.2) (layer "F.Cu") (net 3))
 (segment (start 148.725 66.225) (end 150 67.5) (width 0.2) (layer "F.Cu") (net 3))
 (segment (start 146 66.225) (end 148.725 66.225) (width 0.2) (layer "F.Cu") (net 3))
 (segment (start 154 77) (end 150 73) (width 0.2) (layer "F.Cu") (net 3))
 (segment (start 159.75 83.25) (end 157.75 83.25) (width 0.2) (layer "F.Cu") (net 3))
 (via (at 157.75 83.25) (size 0.6) (drill 0.3) (layers "F.Cu" "B.Cu") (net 3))
 (via (at 154 77) (size 0.6) (drill 0.3) (layers "F.Cu" "B.Cu") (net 3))
 (via (at 159.75 83.25) (size 0.6) (drill 0.3) (layers "F.Cu" "B.Cu") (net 3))
 (segment (start 157.75 83.25) (end 157.649 83.351) (width 0.2) (layer "B.Cu") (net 3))
 (segment (start 159.9125 83.4125) (end 159.75 83.25) (width 0.2) (layer "B.Cu") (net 3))
 (segment (start 157.649 83.351) (end 156.501057 83.351) (width 0.2) (layer "B.Cu") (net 3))
 (segment (start 156.501057 83.351) (end 153.399 80.248943) (width 0.2) (layer "B.Cu") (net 3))
 (segment (start 153.399 78.726) (end 153.80395 78.32105) (width 0.2) (layer "B.Cu") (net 3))
 (segment (start 153.399 80.248943) (end 153.399 78.726) (width 0.2) (layer "B.Cu") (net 3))
 (segment (start 163.25 83.4125) (end 161 83.4125) (width 0.2) (layer "B.Cu") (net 3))
 (segment (start 161 83.45) (end 161 83.4125) (width 0.2) (layer "B.Cu") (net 3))
 (segment (start 154.125 78) (end 154.125 77.125) (width 0.2) (layer "B.Cu") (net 3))
 (segment (start 161 83.4125) (end 159.9125 83.4125) (width 0.2) (layer "B.Cu") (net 3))
 (segment (start 154.125 77.125) (end 154 77) (width 0.2) (layer "B.Cu") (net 3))
 (segment (start 156.5 68.653) (end 156.5 73.727) (width 0.2) (layer "F.Cu") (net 24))
 (segment (start 152.5 68.424998) (end 156.271998 68.424998) (width 0.2) (layer "F.Cu") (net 24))
 (segment (start 162.968 80.195) (end 163.5 80.195) (width 0.2) (layer "F.Cu") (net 24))
 (segment (start 156.271998 68.424998) (end 156.5 68.653) (width 0.2) (layer "F.Cu") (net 24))
 (segment (start 156.5 73.727) (end 162.968 80.195) (width 0.2) (layer "F.Cu") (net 24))
 (via (at 152.5 68.424998) (size 0.6) (drill 0.3) (layers "F.Cu" "B.Cu") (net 24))
 (segment (start 147.5 66.625) (end 149.375 68.5) (width 0.2) (layer "B.Cu") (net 24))
 (segment (start 149.375 68.5) (end 152.5 68.5) (width 0.2) (layer "B.Cu") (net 24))
 (segment (start 152.5 68.5) (end 152.5 68.424998) (width 0.2) (layer "B.Cu") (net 24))
 (segment (start 163.435 63.75) (end 160.75 63.75) (width 0.2) (layer "F.Cu") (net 1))
 (segment (start 149.04 81.445) (end 149.04 80.04) (width 0.2) (layer "F.Cu") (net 1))
 (segment (start 150.5 63.685) (end 152.435 63.685) (width 0.2) (layer "F.Cu") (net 1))
 (segment (start 150 64.185) (end 150.5 63.685) (width 0.2) (layer "F.Cu") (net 1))
 (segment (start 149.04 80.04) (end 149 80) (width 0.2) (layer "F.Cu") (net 1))
 (segment (start 150 64.355) (end 150 64.185) (width 0.2) (layer "F.Cu") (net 1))
 (segment (start 160.75 63.75) (end 152.5 63.75) (width 0.2) (layer "F.Cu") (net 1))
 (segment (start 146 63.685) (end 150.5 63.685) (width 0.2) (layer "F.Cu") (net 1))
 (segment (start 160.25 63.75) (end 160.75 63.75) (width 0.2) (layer "F.Cu") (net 1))
 (segment (start 163.5 63.685) (end 163.435 63.75) (width 0.2) (layer "F.Cu") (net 1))
 (segment (start 152.435 63.685) (end 152.5 63.75) (width 0.2) (layer "F.Cu") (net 1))
 (via (at 150 64.355) (size 0.6) (drill 0.3) (layers "F.Cu" "B.Cu") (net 1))
 (via (at 160.25 63.75) (size 0.6) (drill 0.3) (layers "F.Cu" "B.Cu") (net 1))
 (via (at 149 80) (size 0.6) (drill 0.3) (layers "F.Cu" "B.Cu") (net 1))
 (via (at 152.5 63.75) (size 0.6) (drill 0.3) (layers "F.Cu" "B.Cu") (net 1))
 (segment (start 163.5 85.75) (end 163.5 86.7) (width 0.2) (layer "B.Cu") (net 1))
 (segment (start 146.375 78) (end 146.375 75.5) (width 0.2) (layer "B.Cu") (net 1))
 (segment (start 149.645 64) (end 150 64.355) (width 0.2) (layer "B.Cu") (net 1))
 (segment (start 158.405 85) (end 158.405 82.355) (width 0.2) (layer "B.Cu") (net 1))
 (segment (start 158.405 82.355) (end 156.5 80.45) (width 0.2) (layer "B.Cu") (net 1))
 (segment (start 159 64) (end 160 64) (width 0.2) (layer "B.Cu") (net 1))
 (segment (start 146.375 75.5) (end 147.5 74.375) (width 0.2) (layer "B.Cu") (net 1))
 (segment (start 156.5 80.45) (end 155.25 79.2) (width 0.2) (layer "B.Cu") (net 1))
 (segment (start 153.3075 66.75) (end 153.3075 69.5) (width 0.2) (layer "B.Cu") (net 1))
 (segment (start 149 80) (end 150.565 80) (width 0.2) (layer "B.Cu") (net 1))
 (segment (start 163.5 86.7) (end 163.399 86.801) (width 0.2) (layer "B.Cu") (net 1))
 (segment (start 152.5 65.9425) (end 152.5 63.75) (width 0.2) (layer "B.Cu") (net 1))
 (segment (start 160 64) (end 160.25 63.75) (width 0.2) (layer "B.Cu") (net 1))
 (segment (start 148.375 73.5) (end 153.3075 73.5) (width 0.2) (layer "B.Cu") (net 1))
 (segment (start 158.75 82.01) (end 158.405 82.355) (width 0.2) (layer "B.Cu") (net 1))
 (segment (start 148.5 64) (end 149.645 64) (width 0.2) (layer "B.Cu") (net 1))
 (segment (start 161.2125 80.45) (end 163.25 78.4125) (width 0.2) (layer "B.Cu") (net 1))
 (segment (start 155.25 75.4425) (end 153.3075 73.5) (width 0.2) (layer "B.Cu") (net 1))
 (segment (start 153.3075 72.55) (end 154.07 71.7875) (width 0.2) (layer "B.Cu") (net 1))
 (segment (start 158.75 80.45) (end 161.2125 80.45) (width 0.2) (layer "B.Cu") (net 1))
 (segment (start 159.155 85.75) (end 158.405 85) (width 0.2) (layer "B.Cu") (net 1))
 (segment (start 161 81.55) (end 161 80.6625) (width 0.2) (layer "B.Cu") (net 1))
 (segment (start 158.75 80.45) (end 158.75 82.01) (width 0.2) (layer "B.Cu") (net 1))
 (segment (start 155.25 79.2) (end 155.25 75.4425) (width 0.2) (layer "B.Cu") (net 1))
 (segment (start 163.399 86.801) (end 159.956 86.801) (width 0.2) (layer "B.Cu") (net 1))
 (segment (start 161 80.6625) (end 161.2125 80.45) (width 0.2) (layer "B.Cu") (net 1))
 (segment (start 147.5 74.375) (end 148.375 73.5) (width 0.2) (layer "B.Cu") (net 1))
 (segment (start 154.07 71.7875) (end 154.07 70.2625) (width 0.2) (layer "B.Cu") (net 1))
 (segment (start 154.07 70.2625) (end 153.3075 69.5) (width 0.2) (layer "B.Cu") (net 1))
 (segment (start 153.3075 66.75) (end 152.5 65.9425) (width 0.2) (layer "B.Cu") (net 1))
 (segment (start 150.565 80) (end 153.3075 77.2575) (width 0.2) (layer "B.Cu") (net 1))
 (segment (start 153.3075 72.55) (end 153.3075 73.5) (width 0.2) (layer "B.Cu") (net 1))
 (segment (start 153.3075 73.5) (end 153.3075 77.2575) (width 0.2) (layer "B.Cu") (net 1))
 (segment (start 159.956 86.801) (end 158.905 85.75) (width 0.2) (layer "B.Cu") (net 1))
 (segment (start 161.221 84) (end 161.221 80.394) (width 0.2) (layer "F.Cu") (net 37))
 (segment (start 161.221 85.069) (end 161.221 84) (width 0.2) (layer "F.Cu") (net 37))
 (segment (start 162.25 84.5) (end 161.75 84) (width 0.2) (layer "F.Cu") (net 37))
 (segment (start 161.221 80.394) (end 157.827 77) (width 0.2) (layer "F.Cu") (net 37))
 (segment (start 160.54 85.75) (end 161.221 85.069) (width 0.2) (layer "F.Cu") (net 37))
 (segment (start 157.827 77) (end 156.5 77) (width 0.2) (layer "F.Cu") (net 37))
 (segment (start 161.75 84) (end 161.221 84) (width 0.2) (layer "F.Cu") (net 37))
 (via (at 162.25 84.5) (size 0.6) (drill 0.3) (layers "F.Cu" "B.Cu") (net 37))
 (via (at 156.5 77) (size 0.6) (drill 0.3) (layers "F.Cu" "B.Cu") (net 37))
 (segment (start 156.5 78.55) (end 158.2 76.85) (width 0.2) (layer "B.Cu") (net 37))
 (segment (start 158.2 69.7) (end 154.25 65.75) (width 0.2) (layer "B.Cu") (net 37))
 (segment (start 162.2 85.75) (end 162.2 84.55) (width 0.2) (layer "B.Cu") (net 37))
 (segment (start 162.2 84.55) (end 162.25 84.5) (width 0.2) (layer "B.Cu") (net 37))
 (segment (start 154.25 65.75) (end 153.75 65.75) (width 0.2) (layer "B.Cu") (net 37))
 (segment (start 153.75 65.75) (end 153.75 64) (width 0.2) (layer "B.Cu") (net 37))
 (segment (start 158.2 76.85) (end 158.2 74.4) (width 0.2) (layer "B.Cu") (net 37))
 (segment (start 156.5 77) (end 156.5 78.55) (width 0.2) (layer "B.Cu") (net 37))
 (segment (start 158.2 74.4) (end 158.2 69.7) (width 0.2) (layer "B.Cu") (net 37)))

